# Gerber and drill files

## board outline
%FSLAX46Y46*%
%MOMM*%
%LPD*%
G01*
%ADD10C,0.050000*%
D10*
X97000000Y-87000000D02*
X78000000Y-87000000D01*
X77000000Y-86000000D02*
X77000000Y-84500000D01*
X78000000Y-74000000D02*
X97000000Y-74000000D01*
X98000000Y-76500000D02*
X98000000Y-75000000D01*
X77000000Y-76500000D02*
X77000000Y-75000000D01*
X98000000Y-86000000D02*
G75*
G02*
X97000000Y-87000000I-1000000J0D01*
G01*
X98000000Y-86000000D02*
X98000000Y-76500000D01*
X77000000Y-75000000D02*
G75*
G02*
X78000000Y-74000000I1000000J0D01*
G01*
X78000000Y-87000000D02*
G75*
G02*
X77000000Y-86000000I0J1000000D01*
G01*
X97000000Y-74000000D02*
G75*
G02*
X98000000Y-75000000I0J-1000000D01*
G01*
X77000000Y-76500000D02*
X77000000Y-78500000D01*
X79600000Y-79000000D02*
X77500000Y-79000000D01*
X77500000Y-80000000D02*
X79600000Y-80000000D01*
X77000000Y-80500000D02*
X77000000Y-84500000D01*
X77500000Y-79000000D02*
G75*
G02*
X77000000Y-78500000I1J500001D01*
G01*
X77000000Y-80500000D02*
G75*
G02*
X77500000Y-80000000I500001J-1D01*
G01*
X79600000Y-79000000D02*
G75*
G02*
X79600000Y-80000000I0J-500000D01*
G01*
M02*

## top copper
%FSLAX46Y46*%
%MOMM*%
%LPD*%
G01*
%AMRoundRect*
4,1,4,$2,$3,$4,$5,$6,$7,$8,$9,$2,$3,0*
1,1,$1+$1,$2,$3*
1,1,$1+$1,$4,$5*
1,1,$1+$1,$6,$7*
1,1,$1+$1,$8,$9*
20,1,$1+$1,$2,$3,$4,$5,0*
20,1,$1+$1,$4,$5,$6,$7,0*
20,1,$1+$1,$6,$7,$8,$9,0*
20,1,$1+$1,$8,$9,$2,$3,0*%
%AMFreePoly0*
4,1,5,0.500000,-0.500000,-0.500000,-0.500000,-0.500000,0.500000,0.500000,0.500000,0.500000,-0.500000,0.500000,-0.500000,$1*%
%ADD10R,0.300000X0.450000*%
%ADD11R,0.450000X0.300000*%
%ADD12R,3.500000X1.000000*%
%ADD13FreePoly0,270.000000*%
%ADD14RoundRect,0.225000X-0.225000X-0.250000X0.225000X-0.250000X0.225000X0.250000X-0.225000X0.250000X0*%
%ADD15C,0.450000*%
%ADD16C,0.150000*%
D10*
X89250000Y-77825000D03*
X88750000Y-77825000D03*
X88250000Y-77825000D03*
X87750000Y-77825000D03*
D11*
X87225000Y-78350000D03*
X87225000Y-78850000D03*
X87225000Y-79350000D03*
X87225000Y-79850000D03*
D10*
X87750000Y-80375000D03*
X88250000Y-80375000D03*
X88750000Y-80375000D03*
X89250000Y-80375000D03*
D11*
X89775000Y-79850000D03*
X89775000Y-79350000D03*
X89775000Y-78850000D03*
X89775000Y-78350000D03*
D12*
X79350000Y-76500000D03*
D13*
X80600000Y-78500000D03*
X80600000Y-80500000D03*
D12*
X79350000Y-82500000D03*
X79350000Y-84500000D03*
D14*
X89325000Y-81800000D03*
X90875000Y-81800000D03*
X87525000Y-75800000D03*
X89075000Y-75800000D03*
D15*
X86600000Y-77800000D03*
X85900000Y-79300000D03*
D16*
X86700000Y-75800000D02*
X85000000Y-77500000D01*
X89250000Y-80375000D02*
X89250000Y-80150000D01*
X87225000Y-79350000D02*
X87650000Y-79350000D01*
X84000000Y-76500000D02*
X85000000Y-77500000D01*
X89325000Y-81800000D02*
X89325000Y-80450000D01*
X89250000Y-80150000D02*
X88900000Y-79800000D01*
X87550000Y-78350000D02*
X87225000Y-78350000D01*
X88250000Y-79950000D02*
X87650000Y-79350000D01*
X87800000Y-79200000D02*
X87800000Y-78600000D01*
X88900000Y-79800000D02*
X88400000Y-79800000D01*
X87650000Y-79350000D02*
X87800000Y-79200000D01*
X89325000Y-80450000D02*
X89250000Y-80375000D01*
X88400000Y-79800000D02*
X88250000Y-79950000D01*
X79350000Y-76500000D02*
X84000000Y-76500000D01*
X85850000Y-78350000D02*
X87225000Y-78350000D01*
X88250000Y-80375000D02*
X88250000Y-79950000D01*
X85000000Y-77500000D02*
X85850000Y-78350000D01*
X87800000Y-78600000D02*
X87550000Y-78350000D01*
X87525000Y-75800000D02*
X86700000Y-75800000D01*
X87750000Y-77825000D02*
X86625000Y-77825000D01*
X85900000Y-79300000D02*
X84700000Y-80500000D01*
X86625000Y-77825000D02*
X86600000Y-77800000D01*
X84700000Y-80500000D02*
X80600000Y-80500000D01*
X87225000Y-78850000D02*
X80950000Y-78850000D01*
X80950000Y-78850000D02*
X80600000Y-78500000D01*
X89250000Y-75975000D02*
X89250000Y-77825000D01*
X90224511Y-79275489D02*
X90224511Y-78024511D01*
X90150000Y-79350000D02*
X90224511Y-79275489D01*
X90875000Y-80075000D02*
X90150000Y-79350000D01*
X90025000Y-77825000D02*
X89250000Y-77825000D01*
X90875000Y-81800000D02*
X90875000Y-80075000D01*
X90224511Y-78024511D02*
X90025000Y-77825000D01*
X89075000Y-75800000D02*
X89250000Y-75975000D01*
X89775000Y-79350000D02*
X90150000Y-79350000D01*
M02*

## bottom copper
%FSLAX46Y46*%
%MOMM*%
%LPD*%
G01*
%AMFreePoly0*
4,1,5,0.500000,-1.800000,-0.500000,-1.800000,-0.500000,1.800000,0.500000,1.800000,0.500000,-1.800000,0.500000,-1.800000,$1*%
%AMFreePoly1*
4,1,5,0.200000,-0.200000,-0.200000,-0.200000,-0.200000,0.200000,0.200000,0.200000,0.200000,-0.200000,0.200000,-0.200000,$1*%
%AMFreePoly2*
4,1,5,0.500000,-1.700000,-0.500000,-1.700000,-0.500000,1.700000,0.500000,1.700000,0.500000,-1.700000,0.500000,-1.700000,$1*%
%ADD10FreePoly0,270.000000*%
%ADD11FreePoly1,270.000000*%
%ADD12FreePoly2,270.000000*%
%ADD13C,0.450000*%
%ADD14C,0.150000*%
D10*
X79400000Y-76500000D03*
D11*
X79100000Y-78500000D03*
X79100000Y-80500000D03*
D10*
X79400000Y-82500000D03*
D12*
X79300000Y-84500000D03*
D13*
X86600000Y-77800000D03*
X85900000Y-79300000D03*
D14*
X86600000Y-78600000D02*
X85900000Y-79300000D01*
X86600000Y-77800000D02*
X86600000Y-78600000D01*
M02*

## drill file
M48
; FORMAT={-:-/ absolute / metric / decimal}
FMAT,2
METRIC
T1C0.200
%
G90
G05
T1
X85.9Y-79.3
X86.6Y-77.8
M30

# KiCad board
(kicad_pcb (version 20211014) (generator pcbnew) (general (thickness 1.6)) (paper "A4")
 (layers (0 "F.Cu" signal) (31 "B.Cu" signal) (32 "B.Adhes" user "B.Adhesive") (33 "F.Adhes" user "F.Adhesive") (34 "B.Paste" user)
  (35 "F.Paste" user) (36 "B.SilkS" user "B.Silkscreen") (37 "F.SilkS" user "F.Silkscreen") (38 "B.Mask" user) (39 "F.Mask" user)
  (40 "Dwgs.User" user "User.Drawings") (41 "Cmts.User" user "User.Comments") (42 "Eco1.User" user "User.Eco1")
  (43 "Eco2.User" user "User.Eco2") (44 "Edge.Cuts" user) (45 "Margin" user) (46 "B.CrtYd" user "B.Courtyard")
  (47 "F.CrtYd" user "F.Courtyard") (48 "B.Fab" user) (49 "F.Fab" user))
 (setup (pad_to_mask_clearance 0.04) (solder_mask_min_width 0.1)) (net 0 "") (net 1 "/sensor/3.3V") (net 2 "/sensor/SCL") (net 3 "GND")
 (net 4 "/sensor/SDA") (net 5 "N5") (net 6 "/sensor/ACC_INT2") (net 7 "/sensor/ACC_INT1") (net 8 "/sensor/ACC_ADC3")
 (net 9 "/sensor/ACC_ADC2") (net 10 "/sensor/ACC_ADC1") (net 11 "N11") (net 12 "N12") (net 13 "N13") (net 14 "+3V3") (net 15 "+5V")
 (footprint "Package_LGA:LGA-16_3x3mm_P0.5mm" (layer "F.Cu") (at 88.5 79.1 -90)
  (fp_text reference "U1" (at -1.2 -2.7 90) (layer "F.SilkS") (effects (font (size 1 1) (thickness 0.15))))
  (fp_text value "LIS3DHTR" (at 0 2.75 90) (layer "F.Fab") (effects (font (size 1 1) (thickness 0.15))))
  (pad "1" smd rect (at -1.275 -0.75) (size 0.3 0.45) (layers "F.Cu" "F.Paste" "F.Mask") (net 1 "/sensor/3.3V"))
  (pad "2" smd rect (at -1.275 -0.25) (size 0.3 0.45) (layers "F.Cu" "F.Paste" "F.Mask"))
  (pad "3" smd rect (at -1.275 0.25) (size 0.3 0.45) (layers "F.Cu" "F.Paste" "F.Mask"))
  (pad "4" smd rect (at -1.275 0.75) (size 0.3 0.45) (layers "F.Cu" "F.Paste" "F.Mask") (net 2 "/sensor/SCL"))
  (pad "5" smd rect (at -0.75 1.275 270) (size 0.3 0.45) (layers "F.Cu" "F.Paste" "F.Mask") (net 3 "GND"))
  (pad "6" smd rect (at -0.25 1.275 270) (size 0.3 0.45) (layers "F.Cu" "F.Paste" "F.Mask") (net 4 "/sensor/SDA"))
  (pad "7" smd rect (at 0.25 1.275 270) (size 0.3 0.45) (layers "F.Cu" "F.Paste" "F.Mask") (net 3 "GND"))
  (pad "8" smd rect (at 0.75 1.275 270) (size 0.3 0.45) (layers "F.Cu" "F.Paste" "F.Mask") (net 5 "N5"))
  (pad "9" smd rect (at 1.275 0.75) (size 0.3 0.45) (layers "F.Cu" "F.Paste" "F.Mask") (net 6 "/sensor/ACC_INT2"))
  (pad "10" smd rect (at 1.275 0.25) (size 0.3 0.45) (layers "F.Cu" "F.Paste" "F.Mask") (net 3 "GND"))
  (pad "11" smd rect (at 1.275 -0.25) (size 0.3 0.45) (layers "F.Cu" "F.Paste" "F.Mask") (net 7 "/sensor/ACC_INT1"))
  (pad "12" smd rect (at 1.275 -0.75) (size 0.3 0.45) (layers "F.Cu" "F.Paste" "F.Mask") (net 3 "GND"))
  (pad "13" smd rect (at 0.75 -1.275 270) (size 0.3 0.45) (layers "F.Cu" "F.Paste" "F.Mask") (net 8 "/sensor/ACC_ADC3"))
  (pad "14" smd rect (at 0.25 -1.275 270) (size 0.3 0.45) (layers "F.Cu" "F.Paste" "F.Mask") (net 1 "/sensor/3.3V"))
  (pad "15" smd rect (at -0.25 -1.275 270) (size 0.3 0.45) (layers "F.Cu" "F.Paste" "F.Mask") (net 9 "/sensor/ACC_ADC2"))
  (pad "16" smd rect (at -0.75 -1.275 270) (size 0.3 0.45) (layers "F.Cu" "F.Paste" "F.Mask") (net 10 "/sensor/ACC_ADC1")))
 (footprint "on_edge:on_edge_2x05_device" (layer "F.Cu") (at 77 80.5 -90)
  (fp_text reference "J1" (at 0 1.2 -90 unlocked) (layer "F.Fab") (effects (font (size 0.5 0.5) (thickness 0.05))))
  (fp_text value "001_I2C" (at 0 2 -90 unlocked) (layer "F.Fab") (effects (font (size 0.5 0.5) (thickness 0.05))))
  (fp_line (start -4 0) (end -2 0) (layer "Edge.Cuts") (width 0.05))
  (fp_line (start -1.5 -2.6) (end -1.5 -0.5) (layer "Edge.Cuts") (width 0.05))
  (fp_line (start -0.5 -0.5) (end -0.5 -2.6) (layer "Edge.Cuts") (width 0.05))
  (fp_line (start 0 0) (end 4 0) (layer "Edge.Cuts") (width 0.05))
  (fp_arc (start -1.5 -0.5) (mid -1.646447 -0.146447) (end -2 0) (layer "Edge.Cuts") (width 0.05))
  (fp_arc (start 0 0) (mid -0.353553 -0.146447) (end -0.5 -0.5) (layer "Edge.Cuts") (width 0.05))
  (fp_arc (start -1.5 -2.6) (mid -1 -3.1) (end -0.5 -2.6) (layer "Edge.Cuts") (width 0.05))
  (pad "1" smd rect locked (at -4 -2.35 90) (size 1 3.5) (layers "F.Cu" "F.Mask") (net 3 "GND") (zone_connect 0))
  (pad "2" smd custom locked (at -2 -3.6 270) (size 1 1) (layers "F.Cu" "F.Mask") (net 4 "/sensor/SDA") (zone_connect 0)
   (options (clearance outline) (anchor rect)) (primitives))
  (pad "3" smd custom locked (at 0 -3.6 270) (size 1 1) (layers "F.Cu" "F.Mask") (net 2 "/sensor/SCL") (zone_connect 0)
   (options (clearance outline) (anchor rect)) (primitives))
  (pad "4" smd rect locked (at 2 -2.35 90) (size 1 3.5) (layers "F.Cu" "F.Mask") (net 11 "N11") (zone_connect 0))
  (pad "5" smd rect locked (at 4 -2.35 90) (size 1 3.5) (layers "F.Cu" "F.Mask") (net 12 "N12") (zone_connect 0))
  (pad "6" smd custom locked (at -4 -2.4 270) (size 1 3.6) (layers "B.Cu" "B.Mask") (zone_connect 0)
   (options (clearance outline) (anchor rect)) (primitives))
  (pad "7" smd custom locked (at -2 -2.1 270) (size 0.4 0.4) (layers "B.Cu" "B.Mask") (zone_connect 0)
   (options (clearance outline) (anchor rect)) (primitives))
  (pad "8" smd custom locked (at 0 -2.1 270) (size 0.4 0.4) (layers "B.Cu" "B.Mask") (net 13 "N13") (zone_connect 0)
   (options (clearance outline) (anchor rect)) (primitives))
  (pad "9" smd custom locked (at 2 -2.4 270) (size 1 3.6) (layers "B.Cu" "B.Mask") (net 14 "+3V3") (zone_connect 0)
   (options (clearance outline) (anchor rect)) (primitives))
  (pad "10" smd custom locked (at 4 -2.3 270) (size 1 3.4) (layers "B.Cu" "B.Mask") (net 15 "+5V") (zone_connect 0)
   (options (clearance outline) (anchor rect)) (primitives)))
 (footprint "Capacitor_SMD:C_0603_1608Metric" (layer "F.Cu") (at 90.1 81.8)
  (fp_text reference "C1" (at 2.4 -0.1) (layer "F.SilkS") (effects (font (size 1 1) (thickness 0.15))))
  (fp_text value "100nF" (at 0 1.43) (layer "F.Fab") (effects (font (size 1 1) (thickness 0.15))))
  (pad "1" smd roundrect (at -0.775 0) (size 0.9 0.95) (layers "F.Cu" "F.Paste" "F.Mask") (roundrect_rratio 0.25) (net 3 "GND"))
  (pad "2" smd roundrect (at 0.775 0) (size 0.9 0.95) (layers "F.Cu" "F.Paste" "F.Mask") (roundrect_rratio 0.25) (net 1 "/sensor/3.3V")))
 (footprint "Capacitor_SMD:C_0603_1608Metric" (layer "F.Cu") (at 88.3 75.8)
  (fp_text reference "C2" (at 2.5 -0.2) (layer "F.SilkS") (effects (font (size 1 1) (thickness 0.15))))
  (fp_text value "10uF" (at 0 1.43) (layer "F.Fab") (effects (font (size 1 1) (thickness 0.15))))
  (pad "1" smd roundrect (at -0.775 0) (size 0.9 0.95) (layers "F.Cu" "F.Paste" "F.Mask") (roundrect_rratio 0.25) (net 3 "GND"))
  (pad "2" smd roundrect (at 0.775 0) (size 0.9 0.95) (layers "F.Cu" "F.Paste" "F.Mask") (roundrect_rratio 0.25) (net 1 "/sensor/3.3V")))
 (gr_line (start 97 87) (end 78 87) (layer "Edge.Cuts") (width 0.05))
 (gr_line (start 77 86) (end 77 84.5) (layer "Edge.Cuts") (width 0.05))
 (gr_line (start 78 74) (end 97 74) (layer "Edge.Cuts") (width 0.05))
 (gr_line (start 98 76.5) (end 98 75) (layer "Edge.Cuts") (width 0.05))
 (gr_line (start 77 76.5) (end 77 75) (layer "Edge.Cuts") (width 0.05))
 (gr_arc (start 98 86) (mid 97.707107 86.707107) (end 97 87) (layer "Edge.Cuts") (width 0.05))
 (gr_line (start 98 86) (end 98 76.5) (layer "Edge.Cuts") (width 0.05))
 (gr_arc (start 77 75) (mid 77.292893 74.292893) (end 78 74) (layer "Edge.Cuts") (width 0.05))
 (gr_arc (start 78 87) (mid 77.292893 86.707107) (end 77 86) (layer "Edge.Cuts") (width 0.05))
 (gr_arc (start 97 74) (mid 97.707107 74.292893) (end 98 75) (layer "Edge.Cuts") (width 0.05))
 (segment (start 86.7 75.8) (end 85 77.5) (width 0.15) (layer "F.Cu") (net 3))
 (segment (start 89.25 80.375) (end 89.25 80.15) (width 0.15) (layer "F.Cu") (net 3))
 (segment (start 87.225 79.35) (end 87.65 79.35) (width 0.15) (layer "F.Cu") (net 3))
 (segment (start 84 76.5) (end 85 77.5) (width 0.15) (layer "F.Cu") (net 3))
 (segment (start 89.325 81.8) (end 89.325 80.45) (width 0.15) (layer "F.Cu") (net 3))
 (segment (start 89.25 80.15) (end 88.9 79.8) (width 0.15) (layer "F.Cu") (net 3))
 (segment (start 87.55 78.35) (end 87.225 78.35) (width 0.15) (layer "F.Cu") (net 3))
 (segment (start 88.25 79.95) (end 87.65 79.35) (width 0.15) (layer "F.Cu") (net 3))
 (segment (start 87.8 79.2) (end 87.8 78.6) (width 0.15) (layer "F.Cu") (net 3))
 (segment (start 88.9 79.8) (end 88.4 79.8) (width 0.15) (layer "F.Cu") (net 3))
 (segment (start 87.65 79.35) (end 87.8 79.2) (width 0.15) (layer "F.Cu") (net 3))
 (segment (start 89.325 80.45) (end 89.25 80.375) (width 0.15) (layer "F.Cu") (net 3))
 (segment (start 88.4 79.8) (end 88.25 79.95) (width 0.15) (layer "F.Cu") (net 3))
 (segment (start 79.35 76.5) (end 84 76.5) (width 0.15) (layer "F.Cu") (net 3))
 (segment (start 85.85 78.35) (end 87.225 78.35) (width 0.15) (layer "F.Cu") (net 3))
 (segment (start 88.25 80.375) (end 88.25 79.95) (width 0.15) (layer "F.Cu") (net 3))
 (segment (start 85 77.5) (end 85.85 78.35) (width 0.15) (layer "F.Cu") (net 3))
 (segment (start 87.8 78.6) (end 87.55 78.35) (width 0.15) (layer "F.Cu") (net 3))
 (segment (start 87.525 75.8) (end 86.7 75.8) (width 0.15) (layer "F.Cu") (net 3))
 (segment (start 87.75 77.825) (end 86.625 77.825) (width 0.15) (layer "F.Cu") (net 2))
 (segment (start 85.9 79.3) (end 84.7 80.5) (width 0.15) (layer "F.Cu") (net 2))
 (segment (start 86.625 77.825) (end 86.6 77.8) (width 0.15) (layer "F.Cu") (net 2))
 (segment (start 84.7 80.5) (end 80.6 80.5) (width 0.15) (layer "F.Cu") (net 2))
 (via (at 86.6 77.8) (size 0.45) (drill 0.2) (layers "F.Cu" "B.Cu") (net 2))
 (via (at 85.9 79.3) (size 0.45) (drill 0.2) (layers "F.Cu" "B.Cu") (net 2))
 (segment (start 86.6 78.6) (end 85.9 79.3) (width 0.15) (layer "B.Cu") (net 2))
 (segment (start 86.6 77.8) (end 86.6 78.6) (width 0.15) (layer "B.Cu") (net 2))
 (segment (start 87.225 78.85) (end 80.95 78.85) (width 0.15) (layer "F.Cu") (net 4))
 (segment (start 80.95 78.85) (end 80.6 78.5) (width 0.15) (layer "F.Cu") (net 4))
 (segment (start 89.25 75.975) (end 89.25 77.825) (width 0.15) (layer "F.Cu") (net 1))
 (segment (start 90.224511 79.275489) (end 90.224511 78.024511) (width 0.15) (layer "F.Cu") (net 1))
 (segment (start 90.15 79.35) (end 90.224511 79.275489) (width 0.15) (layer "F.Cu") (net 1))
 (segment (start 90.875 80.075) (end 90.15 79.35) (width 0.15) (layer "F.Cu") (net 1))
 (segment (start 90.025 77.825) (end 89.25 77.825) (width 0.15) (layer "F.Cu") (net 1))
 (segment (start 90.875 81.8) (end 90.875 80.075) (width 0.15) (layer "F.Cu") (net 1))
 (segment (start 90.224511 78.024511) (end 90.025 77.825) (width 0.15) (layer "F.Cu") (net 1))
 (segment (start 89.075 75.8) (end 89.25 75.975) (width 0.15) (layer "F.Cu") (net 1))
 (segment (start 89.775 79.35) (end 90.15 79.35) (width 0.15) (layer "F.Cu") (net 1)))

